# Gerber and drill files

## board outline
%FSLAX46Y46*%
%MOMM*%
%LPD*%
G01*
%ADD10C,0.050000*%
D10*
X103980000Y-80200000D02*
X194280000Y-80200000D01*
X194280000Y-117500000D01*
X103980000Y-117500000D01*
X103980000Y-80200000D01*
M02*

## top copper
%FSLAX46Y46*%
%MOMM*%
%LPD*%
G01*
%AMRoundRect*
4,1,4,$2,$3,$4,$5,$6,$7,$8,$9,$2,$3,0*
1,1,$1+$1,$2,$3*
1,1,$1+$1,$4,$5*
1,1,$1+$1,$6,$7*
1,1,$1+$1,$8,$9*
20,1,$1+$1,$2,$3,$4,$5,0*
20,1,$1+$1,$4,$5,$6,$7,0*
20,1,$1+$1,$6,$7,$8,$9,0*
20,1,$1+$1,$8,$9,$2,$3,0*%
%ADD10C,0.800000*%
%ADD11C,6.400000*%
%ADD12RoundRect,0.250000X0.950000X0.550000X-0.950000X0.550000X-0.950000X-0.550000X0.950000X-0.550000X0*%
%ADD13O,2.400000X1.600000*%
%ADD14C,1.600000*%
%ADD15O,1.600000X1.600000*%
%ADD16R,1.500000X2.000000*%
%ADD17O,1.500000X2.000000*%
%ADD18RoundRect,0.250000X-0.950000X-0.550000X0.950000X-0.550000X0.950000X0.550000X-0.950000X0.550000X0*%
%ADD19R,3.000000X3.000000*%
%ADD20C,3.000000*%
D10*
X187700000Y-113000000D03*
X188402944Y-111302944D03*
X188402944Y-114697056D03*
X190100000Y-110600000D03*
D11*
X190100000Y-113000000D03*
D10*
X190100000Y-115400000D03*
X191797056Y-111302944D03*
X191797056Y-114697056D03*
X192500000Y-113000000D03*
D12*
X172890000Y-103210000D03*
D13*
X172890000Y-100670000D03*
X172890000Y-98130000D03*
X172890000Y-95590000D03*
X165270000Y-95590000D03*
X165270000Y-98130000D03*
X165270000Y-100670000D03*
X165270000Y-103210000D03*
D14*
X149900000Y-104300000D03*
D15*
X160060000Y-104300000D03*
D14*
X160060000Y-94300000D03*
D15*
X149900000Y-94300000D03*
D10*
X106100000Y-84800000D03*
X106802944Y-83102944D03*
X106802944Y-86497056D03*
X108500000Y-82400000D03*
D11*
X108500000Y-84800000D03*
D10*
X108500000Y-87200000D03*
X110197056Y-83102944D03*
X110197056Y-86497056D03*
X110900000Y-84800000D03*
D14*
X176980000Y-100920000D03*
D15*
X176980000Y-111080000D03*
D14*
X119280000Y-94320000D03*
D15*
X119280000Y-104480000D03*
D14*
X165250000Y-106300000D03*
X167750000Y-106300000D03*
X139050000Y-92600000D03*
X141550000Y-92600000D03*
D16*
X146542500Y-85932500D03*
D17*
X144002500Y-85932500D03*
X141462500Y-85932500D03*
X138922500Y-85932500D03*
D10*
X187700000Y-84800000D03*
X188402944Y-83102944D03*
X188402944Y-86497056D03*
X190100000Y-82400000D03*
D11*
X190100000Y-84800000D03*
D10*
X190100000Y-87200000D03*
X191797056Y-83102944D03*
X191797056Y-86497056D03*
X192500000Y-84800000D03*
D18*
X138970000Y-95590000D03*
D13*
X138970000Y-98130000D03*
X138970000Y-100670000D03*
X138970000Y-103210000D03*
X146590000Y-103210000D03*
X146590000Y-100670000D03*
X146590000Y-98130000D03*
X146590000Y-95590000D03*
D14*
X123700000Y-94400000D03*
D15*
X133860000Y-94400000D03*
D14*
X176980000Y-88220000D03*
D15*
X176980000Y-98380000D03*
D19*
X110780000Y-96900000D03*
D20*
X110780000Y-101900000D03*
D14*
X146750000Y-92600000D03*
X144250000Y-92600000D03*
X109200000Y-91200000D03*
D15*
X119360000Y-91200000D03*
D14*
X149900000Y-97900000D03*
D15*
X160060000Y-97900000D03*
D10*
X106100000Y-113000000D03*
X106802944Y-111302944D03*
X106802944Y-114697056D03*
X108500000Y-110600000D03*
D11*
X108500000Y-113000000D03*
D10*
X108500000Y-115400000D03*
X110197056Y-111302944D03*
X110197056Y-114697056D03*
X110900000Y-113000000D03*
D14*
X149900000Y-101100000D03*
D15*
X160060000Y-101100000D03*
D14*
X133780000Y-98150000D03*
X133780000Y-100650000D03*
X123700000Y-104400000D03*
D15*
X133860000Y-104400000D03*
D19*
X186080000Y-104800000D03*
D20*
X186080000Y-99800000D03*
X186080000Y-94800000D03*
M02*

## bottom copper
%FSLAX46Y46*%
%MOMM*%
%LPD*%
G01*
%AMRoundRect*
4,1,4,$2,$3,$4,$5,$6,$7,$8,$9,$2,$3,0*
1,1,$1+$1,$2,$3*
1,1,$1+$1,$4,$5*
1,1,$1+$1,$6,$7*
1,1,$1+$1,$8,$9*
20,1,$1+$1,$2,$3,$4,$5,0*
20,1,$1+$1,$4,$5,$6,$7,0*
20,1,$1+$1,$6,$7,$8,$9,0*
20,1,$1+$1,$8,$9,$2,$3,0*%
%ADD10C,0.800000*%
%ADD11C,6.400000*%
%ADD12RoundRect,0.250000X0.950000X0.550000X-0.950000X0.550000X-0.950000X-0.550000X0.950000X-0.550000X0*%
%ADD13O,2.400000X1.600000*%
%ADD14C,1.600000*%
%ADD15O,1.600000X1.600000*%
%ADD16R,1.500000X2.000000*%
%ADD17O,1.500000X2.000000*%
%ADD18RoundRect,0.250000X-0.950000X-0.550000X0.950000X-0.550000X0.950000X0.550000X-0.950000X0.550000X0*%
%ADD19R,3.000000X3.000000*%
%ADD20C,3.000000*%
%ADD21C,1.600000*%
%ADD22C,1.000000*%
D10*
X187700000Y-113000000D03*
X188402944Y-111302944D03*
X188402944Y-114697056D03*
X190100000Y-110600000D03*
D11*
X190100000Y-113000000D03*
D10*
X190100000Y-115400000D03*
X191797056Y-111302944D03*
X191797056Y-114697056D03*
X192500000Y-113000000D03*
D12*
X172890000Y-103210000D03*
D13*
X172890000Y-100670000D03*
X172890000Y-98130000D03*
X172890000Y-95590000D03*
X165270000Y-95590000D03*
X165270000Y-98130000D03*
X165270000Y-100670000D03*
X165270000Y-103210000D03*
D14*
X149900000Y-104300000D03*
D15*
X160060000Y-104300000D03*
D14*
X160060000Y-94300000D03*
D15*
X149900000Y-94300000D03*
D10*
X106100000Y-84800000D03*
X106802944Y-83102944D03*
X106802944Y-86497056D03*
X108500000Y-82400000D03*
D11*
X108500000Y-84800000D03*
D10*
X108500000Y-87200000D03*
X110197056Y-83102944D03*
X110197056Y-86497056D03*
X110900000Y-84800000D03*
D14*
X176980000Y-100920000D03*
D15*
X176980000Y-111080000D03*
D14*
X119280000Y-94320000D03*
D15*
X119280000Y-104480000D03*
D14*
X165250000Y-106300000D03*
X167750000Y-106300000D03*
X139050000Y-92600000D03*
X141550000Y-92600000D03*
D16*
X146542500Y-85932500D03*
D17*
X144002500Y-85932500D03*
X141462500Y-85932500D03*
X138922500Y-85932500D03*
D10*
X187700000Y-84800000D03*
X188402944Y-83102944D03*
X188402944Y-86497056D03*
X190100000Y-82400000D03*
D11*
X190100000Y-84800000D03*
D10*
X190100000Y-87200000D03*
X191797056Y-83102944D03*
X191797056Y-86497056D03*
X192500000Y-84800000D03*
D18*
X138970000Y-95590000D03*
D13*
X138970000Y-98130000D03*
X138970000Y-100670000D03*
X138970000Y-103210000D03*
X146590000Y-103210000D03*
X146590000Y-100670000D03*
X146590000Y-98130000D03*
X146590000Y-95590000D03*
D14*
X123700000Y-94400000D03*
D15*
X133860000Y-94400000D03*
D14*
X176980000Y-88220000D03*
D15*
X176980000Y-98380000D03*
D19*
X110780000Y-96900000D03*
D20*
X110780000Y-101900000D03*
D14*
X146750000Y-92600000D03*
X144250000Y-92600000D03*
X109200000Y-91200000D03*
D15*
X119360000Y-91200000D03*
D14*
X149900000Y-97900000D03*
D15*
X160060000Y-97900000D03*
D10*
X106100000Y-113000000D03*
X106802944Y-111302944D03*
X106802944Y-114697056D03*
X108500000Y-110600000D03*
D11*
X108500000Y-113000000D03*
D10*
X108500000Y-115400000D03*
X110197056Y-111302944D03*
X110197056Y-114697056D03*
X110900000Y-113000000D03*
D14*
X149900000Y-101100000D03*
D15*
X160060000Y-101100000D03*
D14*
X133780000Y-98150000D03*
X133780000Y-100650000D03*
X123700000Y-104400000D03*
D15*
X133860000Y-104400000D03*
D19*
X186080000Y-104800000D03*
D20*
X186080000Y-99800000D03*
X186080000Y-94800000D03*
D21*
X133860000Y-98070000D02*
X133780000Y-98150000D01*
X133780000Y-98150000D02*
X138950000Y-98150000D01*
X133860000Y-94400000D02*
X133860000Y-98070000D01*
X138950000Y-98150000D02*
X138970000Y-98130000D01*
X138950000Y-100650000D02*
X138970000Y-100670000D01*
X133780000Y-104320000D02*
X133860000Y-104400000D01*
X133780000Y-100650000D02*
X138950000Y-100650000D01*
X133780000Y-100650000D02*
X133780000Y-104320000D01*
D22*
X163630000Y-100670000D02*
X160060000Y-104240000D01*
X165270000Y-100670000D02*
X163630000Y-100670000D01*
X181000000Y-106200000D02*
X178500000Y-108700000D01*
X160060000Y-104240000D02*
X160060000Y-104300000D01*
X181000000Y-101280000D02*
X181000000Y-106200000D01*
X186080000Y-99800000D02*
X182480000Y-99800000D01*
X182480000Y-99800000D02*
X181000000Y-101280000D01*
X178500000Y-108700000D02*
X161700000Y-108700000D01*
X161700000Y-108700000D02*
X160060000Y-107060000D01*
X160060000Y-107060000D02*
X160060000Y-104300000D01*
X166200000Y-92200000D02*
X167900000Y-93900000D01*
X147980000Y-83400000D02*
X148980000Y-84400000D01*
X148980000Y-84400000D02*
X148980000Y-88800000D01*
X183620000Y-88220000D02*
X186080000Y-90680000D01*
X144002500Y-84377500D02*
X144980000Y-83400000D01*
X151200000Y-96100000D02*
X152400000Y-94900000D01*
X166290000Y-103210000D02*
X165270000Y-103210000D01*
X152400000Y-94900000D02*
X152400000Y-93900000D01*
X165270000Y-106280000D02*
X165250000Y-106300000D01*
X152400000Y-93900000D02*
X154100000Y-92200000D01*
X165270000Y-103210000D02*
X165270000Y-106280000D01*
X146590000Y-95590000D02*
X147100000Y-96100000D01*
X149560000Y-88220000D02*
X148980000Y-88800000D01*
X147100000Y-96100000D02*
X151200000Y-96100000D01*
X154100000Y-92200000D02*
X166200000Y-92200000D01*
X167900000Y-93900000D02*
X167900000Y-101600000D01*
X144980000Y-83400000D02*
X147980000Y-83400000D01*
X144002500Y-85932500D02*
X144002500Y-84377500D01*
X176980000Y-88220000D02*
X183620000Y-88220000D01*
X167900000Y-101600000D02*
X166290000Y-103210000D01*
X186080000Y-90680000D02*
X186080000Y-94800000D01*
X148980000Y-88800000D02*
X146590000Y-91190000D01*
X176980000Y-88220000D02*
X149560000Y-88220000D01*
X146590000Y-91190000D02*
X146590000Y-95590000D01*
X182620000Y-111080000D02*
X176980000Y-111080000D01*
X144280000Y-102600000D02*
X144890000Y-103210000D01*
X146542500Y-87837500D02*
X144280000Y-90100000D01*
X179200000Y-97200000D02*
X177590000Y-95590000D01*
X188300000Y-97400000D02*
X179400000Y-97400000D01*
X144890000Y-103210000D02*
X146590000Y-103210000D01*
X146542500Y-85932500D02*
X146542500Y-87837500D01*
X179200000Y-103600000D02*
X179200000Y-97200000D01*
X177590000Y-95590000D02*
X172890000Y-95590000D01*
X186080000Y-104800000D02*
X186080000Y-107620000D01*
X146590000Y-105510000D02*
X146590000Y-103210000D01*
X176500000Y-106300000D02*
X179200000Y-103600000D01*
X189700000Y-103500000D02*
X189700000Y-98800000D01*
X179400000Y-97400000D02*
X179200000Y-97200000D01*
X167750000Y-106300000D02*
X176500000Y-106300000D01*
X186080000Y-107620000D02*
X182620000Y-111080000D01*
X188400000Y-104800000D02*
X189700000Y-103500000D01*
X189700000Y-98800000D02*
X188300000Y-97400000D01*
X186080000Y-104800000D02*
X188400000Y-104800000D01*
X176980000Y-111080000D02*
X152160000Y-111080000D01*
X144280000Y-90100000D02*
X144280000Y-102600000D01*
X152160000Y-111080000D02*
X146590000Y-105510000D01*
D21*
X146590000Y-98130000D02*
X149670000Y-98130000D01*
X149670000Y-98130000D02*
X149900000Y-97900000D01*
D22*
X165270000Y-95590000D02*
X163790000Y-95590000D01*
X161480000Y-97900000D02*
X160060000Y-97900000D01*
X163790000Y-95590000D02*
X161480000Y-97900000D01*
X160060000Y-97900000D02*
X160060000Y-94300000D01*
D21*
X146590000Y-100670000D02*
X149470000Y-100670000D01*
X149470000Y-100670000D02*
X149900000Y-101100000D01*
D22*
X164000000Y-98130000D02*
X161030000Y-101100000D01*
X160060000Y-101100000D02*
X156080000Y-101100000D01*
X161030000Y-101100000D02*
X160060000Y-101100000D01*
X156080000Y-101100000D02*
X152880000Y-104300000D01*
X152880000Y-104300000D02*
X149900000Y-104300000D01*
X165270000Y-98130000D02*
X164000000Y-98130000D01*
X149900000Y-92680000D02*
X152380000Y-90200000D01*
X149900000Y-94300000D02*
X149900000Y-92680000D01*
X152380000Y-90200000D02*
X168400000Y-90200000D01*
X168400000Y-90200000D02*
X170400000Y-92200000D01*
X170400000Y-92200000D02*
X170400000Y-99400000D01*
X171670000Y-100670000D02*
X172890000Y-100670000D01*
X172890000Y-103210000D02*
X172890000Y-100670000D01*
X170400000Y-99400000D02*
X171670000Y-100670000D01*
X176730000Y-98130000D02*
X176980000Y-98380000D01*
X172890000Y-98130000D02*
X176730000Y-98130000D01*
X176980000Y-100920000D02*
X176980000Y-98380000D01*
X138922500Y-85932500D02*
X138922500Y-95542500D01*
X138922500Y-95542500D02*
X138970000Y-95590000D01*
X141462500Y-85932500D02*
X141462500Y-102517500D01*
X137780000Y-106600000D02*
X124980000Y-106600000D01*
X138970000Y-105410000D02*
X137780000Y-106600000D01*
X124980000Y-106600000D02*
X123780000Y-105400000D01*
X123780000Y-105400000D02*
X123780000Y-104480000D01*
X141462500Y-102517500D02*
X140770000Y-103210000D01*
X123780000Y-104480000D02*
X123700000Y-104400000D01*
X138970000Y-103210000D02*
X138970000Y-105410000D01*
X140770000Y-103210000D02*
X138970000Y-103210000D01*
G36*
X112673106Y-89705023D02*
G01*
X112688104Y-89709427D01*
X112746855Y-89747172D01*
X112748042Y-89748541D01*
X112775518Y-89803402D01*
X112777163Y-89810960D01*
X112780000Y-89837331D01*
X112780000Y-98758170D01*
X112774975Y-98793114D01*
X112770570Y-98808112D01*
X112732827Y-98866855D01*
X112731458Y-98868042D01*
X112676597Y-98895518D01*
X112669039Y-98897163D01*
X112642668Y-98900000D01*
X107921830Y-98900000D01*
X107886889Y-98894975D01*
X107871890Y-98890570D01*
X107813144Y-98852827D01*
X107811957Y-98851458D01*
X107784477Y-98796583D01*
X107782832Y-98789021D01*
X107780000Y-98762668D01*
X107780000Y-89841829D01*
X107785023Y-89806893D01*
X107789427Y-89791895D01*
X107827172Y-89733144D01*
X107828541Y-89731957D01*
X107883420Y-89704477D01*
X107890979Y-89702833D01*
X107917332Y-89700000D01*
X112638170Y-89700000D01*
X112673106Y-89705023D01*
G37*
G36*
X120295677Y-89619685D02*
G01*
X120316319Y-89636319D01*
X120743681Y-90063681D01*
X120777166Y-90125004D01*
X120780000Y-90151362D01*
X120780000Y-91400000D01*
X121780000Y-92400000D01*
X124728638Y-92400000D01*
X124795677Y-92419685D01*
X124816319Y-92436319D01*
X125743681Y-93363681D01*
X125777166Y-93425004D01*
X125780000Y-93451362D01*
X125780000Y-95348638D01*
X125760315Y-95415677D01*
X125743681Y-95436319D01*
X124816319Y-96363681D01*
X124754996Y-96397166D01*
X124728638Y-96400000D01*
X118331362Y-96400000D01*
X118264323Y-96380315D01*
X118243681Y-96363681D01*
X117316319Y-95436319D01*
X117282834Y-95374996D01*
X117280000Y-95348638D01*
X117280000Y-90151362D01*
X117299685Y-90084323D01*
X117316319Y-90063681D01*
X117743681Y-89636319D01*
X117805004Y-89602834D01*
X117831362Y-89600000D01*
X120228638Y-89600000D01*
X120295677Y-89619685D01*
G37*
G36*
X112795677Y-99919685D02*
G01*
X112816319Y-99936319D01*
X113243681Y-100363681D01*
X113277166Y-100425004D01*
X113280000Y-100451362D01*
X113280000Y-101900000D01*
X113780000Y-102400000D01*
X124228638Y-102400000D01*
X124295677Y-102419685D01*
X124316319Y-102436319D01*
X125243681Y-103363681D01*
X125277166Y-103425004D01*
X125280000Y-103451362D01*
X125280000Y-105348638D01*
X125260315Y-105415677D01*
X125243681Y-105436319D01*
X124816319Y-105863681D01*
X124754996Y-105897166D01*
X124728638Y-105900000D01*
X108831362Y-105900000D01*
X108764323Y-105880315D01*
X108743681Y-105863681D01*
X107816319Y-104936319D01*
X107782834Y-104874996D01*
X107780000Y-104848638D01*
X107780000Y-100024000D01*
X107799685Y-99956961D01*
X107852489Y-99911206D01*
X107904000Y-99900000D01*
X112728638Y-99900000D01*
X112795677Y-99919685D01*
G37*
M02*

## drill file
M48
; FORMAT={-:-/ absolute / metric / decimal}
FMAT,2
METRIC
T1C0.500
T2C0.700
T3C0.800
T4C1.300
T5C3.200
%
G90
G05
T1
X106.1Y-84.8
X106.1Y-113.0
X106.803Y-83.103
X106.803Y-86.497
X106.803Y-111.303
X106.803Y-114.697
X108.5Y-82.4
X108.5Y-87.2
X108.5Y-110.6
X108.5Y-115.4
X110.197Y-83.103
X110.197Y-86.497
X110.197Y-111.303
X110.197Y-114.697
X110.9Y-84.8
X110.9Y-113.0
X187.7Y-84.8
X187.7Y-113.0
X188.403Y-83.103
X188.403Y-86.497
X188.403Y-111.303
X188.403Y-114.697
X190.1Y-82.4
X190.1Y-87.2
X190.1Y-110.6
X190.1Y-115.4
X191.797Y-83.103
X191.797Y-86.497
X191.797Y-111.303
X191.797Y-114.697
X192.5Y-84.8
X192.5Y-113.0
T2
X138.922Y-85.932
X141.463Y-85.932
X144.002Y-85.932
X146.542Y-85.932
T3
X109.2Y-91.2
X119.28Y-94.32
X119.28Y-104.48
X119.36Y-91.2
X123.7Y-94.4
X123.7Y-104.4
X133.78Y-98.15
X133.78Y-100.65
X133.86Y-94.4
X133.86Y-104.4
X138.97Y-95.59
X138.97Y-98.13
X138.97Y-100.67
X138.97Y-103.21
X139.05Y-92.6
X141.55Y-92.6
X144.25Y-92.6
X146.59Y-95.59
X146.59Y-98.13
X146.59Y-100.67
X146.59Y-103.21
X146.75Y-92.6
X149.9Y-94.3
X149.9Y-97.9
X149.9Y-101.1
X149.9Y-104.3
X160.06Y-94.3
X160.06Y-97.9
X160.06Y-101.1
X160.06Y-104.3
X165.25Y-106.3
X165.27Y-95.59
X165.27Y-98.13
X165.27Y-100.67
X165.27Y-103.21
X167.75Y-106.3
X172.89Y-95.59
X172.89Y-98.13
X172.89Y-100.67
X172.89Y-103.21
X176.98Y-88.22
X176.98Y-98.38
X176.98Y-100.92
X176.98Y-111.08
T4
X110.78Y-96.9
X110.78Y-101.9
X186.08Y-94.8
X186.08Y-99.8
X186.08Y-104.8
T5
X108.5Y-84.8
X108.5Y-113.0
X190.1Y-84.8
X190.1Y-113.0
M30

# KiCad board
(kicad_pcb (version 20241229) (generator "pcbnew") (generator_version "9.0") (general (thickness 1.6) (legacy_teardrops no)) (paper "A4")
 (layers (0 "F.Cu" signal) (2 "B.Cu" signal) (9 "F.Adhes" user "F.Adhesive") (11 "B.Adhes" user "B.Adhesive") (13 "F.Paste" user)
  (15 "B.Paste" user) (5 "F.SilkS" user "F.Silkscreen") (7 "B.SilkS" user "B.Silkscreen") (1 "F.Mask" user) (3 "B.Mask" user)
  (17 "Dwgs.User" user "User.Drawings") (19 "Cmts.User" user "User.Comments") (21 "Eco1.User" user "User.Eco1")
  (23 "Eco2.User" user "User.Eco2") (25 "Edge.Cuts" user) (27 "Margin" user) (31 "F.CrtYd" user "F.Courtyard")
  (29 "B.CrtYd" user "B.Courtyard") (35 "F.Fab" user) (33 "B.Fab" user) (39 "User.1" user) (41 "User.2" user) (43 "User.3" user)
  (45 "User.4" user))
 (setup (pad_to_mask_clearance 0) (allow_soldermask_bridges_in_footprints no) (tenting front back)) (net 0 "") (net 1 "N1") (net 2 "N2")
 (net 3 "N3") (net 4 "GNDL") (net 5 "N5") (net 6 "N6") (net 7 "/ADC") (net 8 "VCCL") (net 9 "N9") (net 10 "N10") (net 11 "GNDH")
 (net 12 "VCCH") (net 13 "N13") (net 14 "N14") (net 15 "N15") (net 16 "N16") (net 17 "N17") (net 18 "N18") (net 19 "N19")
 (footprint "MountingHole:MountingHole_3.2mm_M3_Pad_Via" (layer "F.Cu") (at 190.1 113)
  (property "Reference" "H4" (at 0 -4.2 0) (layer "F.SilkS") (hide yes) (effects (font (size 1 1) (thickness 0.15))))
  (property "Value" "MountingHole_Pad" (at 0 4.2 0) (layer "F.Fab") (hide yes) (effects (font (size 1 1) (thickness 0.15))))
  (pad "1" thru_hole circle (at -2.4 0) (size 0.8 0.8) (drill 0.5) (layers "*.Cu" "*.Mask") (remove_unused_layers no) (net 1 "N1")
   (zone_connect 2))
  (pad "1" thru_hole circle (at -1.697056 -1.697056) (size 0.8 0.8) (drill 0.5) (layers "*.Cu" "*.Mask") (remove_unused_layers no)
   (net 1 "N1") (zone_connect 2))
  (pad "1" thru_hole circle (at -1.697056 1.697056) (size 0.8 0.8) (drill 0.5) (layers "*.Cu" "*.Mask") (remove_unused_layers no)
   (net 1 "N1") (zone_connect 2))
  (pad "1" thru_hole circle (at 0 -2.4) (size 0.8 0.8) (drill 0.5) (layers "*.Cu" "*.Mask") (remove_unused_layers no) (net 1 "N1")
   (zone_connect 2))
  (pad "1" thru_hole circle (at 0 0) (size 6.4 6.4) (drill 3.2) (layers "*.Cu" "*.Mask") (remove_unused_layers no) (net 1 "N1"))
  (pad "1" thru_hole circle (at 0 2.4) (size 0.8 0.8) (drill 0.5) (layers "*.Cu" "*.Mask") (remove_unused_layers no) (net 1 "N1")
   (zone_connect 2))
  (pad "1" thru_hole circle (at 1.697056 -1.697056) (size 0.8 0.8) (drill 0.5) (layers "*.Cu" "*.Mask") (remove_unused_layers no)
   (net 1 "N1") (zone_connect 2))
  (pad "1" thru_hole circle (at 1.697056 1.697056) (size 0.8 0.8) (drill 0.5) (layers "*.Cu" "*.Mask") (remove_unused_layers no)
   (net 1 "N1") (zone_connect 2))
  (pad "1" thru_hole circle (at 2.4 0) (size 0.8 0.8) (drill 0.5) (layers "*.Cu" "*.Mask") (remove_unused_layers no) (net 1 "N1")
   (zone_connect 2)))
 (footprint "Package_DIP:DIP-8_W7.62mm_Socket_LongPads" (layer "F.Cu") (at 172.89 103.21 180)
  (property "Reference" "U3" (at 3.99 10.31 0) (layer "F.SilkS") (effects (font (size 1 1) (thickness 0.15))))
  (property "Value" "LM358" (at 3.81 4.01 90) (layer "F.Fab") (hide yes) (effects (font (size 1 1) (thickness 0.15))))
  (pad "1" thru_hole roundrect (at 0 0 180) (size 2.4 1.6) (drill 0.8) (layers "*.Cu" "*.Mask") (remove_unused_layers no)
   (roundrect_rratio 0.15625) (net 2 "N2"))
  (pad "2" thru_hole oval (at 0 2.54 180) (size 2.4 1.6) (drill 0.8) (layers "*.Cu" "*.Mask") (remove_unused_layers no) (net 2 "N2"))
  (pad "3" thru_hole oval (at 0 5.08 180) (size 2.4 1.6) (drill 0.8) (layers "*.Cu" "*.Mask") (remove_unused_layers no) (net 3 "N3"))
  (pad "4" thru_hole oval (at 0 7.62 180) (size 2.4 1.6) (drill 0.8) (layers "*.Cu" "*.Mask") (remove_unused_layers no) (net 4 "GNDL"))
  (pad "5" thru_hole oval (at 7.62 7.62 180) (size 2.4 1.6) (drill 0.8) (layers "*.Cu" "*.Mask") (remove_unused_layers no) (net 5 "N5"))
  (pad "6" thru_hole oval (at 7.62 5.08 180) (size 2.4 1.6) (drill 0.8) (layers "*.Cu" "*.Mask") (remove_unused_layers no) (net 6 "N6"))
  (pad "7" thru_hole oval (at 7.62 2.54 180) (size 2.4 1.6) (drill 0.8) (layers "*.Cu" "*.Mask") (remove_unused_layers no) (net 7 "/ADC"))
  (pad "8" thru_hole oval (at 7.62 0 180) (size 2.4 1.6) (drill 0.8) (layers "*.Cu" "*.Mask") (remove_unused_layers no) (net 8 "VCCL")))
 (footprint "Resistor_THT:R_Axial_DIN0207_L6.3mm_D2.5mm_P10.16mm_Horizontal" (layer "F.Cu") (at 149.9 104.3)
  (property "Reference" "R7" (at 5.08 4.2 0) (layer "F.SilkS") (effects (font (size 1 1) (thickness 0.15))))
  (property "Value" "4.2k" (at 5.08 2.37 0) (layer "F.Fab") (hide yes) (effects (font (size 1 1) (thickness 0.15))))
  (pad "1" thru_hole circle (at 0 0) (size 1.6 1.6) (drill 0.8) (layers "*.Cu" "*.Mask") (remove_unused_layers no) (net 6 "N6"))
  (pad "2" thru_hole oval (at 10.16 0) (size 1.6 1.6) (drill 0.8) (layers "*.Cu" "*.Mask") (remove_unused_layers no) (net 7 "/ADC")))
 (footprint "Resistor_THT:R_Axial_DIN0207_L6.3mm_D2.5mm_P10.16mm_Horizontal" (layer "F.Cu") (at 160.06 94.3 180)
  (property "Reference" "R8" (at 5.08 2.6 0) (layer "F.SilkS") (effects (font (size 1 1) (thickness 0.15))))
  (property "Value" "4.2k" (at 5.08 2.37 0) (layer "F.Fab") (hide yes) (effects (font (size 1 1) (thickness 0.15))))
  (pad "1" thru_hole circle (at 0 0 180) (size 1.6 1.6) (drill 0.8) (layers "*.Cu" "*.Mask") (remove_unused_layers no) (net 5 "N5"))
  (pad "2" thru_hole oval (at 10.16 0 180) (size 1.6 1.6) (drill 0.8) (layers "*.Cu" "*.Mask") (remove_unused_layers no) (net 2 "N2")))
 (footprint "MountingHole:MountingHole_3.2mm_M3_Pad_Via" (layer "F.Cu") (at 108.5 84.8)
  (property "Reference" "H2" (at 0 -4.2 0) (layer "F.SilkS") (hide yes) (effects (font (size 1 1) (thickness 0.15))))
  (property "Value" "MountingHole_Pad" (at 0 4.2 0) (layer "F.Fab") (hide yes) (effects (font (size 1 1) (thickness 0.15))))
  (pad "1" thru_hole circle (at -2.4 0) (size 0.8 0.8) (drill 0.5) (layers "*.Cu" "*.Mask") (remove_unused_layers no) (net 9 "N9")
   (zone_connect 2))
  (pad "1" thru_hole circle (at -1.697056 -1.697056) (size 0.8 0.8) (drill 0.5) (layers "*.Cu" "*.Mask") (remove_unused_layers no)
   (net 9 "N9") (zone_connect 2))
  (pad "1" thru_hole circle (at -1.697056 1.697056) (size 0.8 0.8) (drill 0.5) (layers "*.Cu" "*.Mask") (remove_unused_layers no)
   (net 9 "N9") (zone_connect 2))
  (pad "1" thru_hole circle (at 0 -2.4) (size 0.8 0.8) (drill 0.5) (layers "*.Cu" "*.Mask") (remove_unused_layers no) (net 9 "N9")
   (zone_connect 2))
  (pad "1" thru_hole circle (at 0 0) (size 6.4 6.4) (drill 3.2) (layers "*.Cu" "*.Mask") (remove_unused_layers no) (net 9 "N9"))
  (pad "1" thru_hole circle (at 0 2.4) (size 0.8 0.8) (drill 0.5) (layers "*.Cu" "*.Mask") (remove_unused_layers no) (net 9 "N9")
   (zone_connect 2))
  (pad "1" thru_hole circle (at 1.697056 -1.697056) (size 0.8 0.8) (drill 0.5) (layers "*.Cu" "*.Mask") (remove_unused_layers no)
   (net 9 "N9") (zone_connect 2))
  (pad "1" thru_hole circle (at 1.697056 1.697056) (size 0.8 0.8) (drill 0.5) (layers "*.Cu" "*.Mask") (remove_unused_layers no)
   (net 9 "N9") (zone_connect 2))
  (pad "1" thru_hole circle (at 2.4 0) (size 0.8 0.8) (drill 0.5) (layers "*.Cu" "*.Mask") (remove_unused_layers no) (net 9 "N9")
   (zone_connect 2)))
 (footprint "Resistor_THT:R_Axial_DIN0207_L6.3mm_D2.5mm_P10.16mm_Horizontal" (layer "F.Cu") (at 176.98 100.92 -90)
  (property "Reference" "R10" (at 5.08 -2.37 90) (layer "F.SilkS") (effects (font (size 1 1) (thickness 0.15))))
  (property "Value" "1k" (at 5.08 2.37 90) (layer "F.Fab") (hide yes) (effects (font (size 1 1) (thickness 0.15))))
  (pad "1" thru_hole circle (at 0 0 270) (size 1.6 1.6) (drill 0.8) (layers "*.Cu" "*.Mask") (remove_unused_layers no) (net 3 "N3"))
  (pad "2" thru_hole oval (at 10.16 0 270) (size 1.6 1.6) (drill 0.8) (layers "*.Cu" "*.Mask") (remove_unused_layers no) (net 4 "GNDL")))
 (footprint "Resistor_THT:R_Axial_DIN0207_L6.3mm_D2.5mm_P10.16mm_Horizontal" (layer "F.Cu") (at 119.28 94.32 -90)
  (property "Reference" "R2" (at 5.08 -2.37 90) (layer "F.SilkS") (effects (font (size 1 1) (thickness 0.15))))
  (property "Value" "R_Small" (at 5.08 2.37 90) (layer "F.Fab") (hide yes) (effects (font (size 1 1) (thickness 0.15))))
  (pad "1" thru_hole circle (at 0 0 270) (size 1.6 1.6) (drill 0.8) (layers "*.Cu" "*.Mask") (remove_unused_layers no) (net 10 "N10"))
  (pad "2" thru_hole oval (at 10.16 0 270) (size 1.6 1.6) (drill 0.8) (layers "*.Cu" "*.Mask") (remove_unused_layers no) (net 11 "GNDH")))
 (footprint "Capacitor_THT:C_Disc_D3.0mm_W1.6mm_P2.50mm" (layer "F.Cu") (at 165.25 106.3)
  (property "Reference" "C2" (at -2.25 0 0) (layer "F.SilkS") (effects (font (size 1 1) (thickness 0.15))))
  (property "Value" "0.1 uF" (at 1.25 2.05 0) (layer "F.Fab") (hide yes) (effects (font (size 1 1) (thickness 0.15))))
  (pad "1" thru_hole circle (at 0 0) (size 1.6 1.6) (drill 0.8) (layers "*.Cu" "*.Mask") (remove_unused_layers no) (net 8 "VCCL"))
  (pad "2" thru_hole circle (at 2.5 0) (size 1.6 1.6) (drill 0.8) (layers "*.Cu" "*.Mask") (remove_unused_layers no) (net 4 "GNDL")))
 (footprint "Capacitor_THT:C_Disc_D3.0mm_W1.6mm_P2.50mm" (layer "F.Cu") (at 139.05 92.6)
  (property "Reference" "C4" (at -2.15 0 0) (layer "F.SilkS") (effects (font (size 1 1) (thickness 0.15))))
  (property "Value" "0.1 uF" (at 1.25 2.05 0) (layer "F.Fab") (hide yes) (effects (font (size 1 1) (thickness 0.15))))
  (pad "1" thru_hole circle (at 0 0) (size 1.6 1.6) (drill 0.8) (layers "*.Cu" "*.Mask") (remove_unused_layers no) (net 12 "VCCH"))
  (pad "2" thru_hole circle (at 2.5 0) (size 1.6 1.6) (drill 0.8) (layers "*.Cu" "*.Mask") (remove_unused_layers no) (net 11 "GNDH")))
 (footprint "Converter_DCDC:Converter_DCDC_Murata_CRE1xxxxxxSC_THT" (layer "F.Cu") (at 146.5425 85.9325 -90)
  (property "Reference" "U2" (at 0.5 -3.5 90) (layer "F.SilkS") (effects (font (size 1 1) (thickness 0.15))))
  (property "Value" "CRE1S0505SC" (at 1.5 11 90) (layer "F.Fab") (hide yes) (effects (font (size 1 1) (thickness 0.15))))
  (pad "1" thru_hole rect (at 0 0 180) (size 1.5 2) (drill 0.7) (layers "*.Cu" "*.Mask") (remove_unused_layers no) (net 4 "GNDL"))
  (pad "2" thru_hole oval (at 0 2.54 180) (size 1.5 2) (drill 0.7) (layers "*.Cu" "*.Mask") (remove_unused_layers no) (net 8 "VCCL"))
  (pad "3" thru_hole oval (at 0 5.08 180) (size 1.5 2) (drill 0.7) (layers "*.Cu" "*.Mask") (remove_unused_layers no) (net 11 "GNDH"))
  (pad "4" thru_hole oval (at 0 7.62 180) (size 1.5 2) (drill 0.7) (layers "*.Cu" "*.Mask") (remove_unused_layers no) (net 12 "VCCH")))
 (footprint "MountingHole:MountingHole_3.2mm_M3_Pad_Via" (layer "F.Cu") (at 190.1 84.8)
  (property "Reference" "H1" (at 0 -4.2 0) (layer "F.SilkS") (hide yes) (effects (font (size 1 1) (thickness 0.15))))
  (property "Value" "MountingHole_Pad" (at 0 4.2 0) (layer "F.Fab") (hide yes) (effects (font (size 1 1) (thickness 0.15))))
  (pad "1" thru_hole circle (at -2.4 0) (size 0.8 0.8) (drill 0.5) (layers "*.Cu" "*.Mask") (remove_unused_layers no) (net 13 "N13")
   (zone_connect 2))
  (pad "1" thru_hole circle (at -1.697056 -1.697056) (size 0.8 0.8) (drill 0.5) (layers "*.Cu" "*.Mask") (remove_unused_layers no)
   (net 13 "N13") (zone_connect 2))
  (pad "1" thru_hole circle (at -1.697056 1.697056) (size 0.8 0.8) (drill 0.5) (layers "*.Cu" "*.Mask") (remove_unused_layers no)
   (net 13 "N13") (zone_connect 2))
  (pad "1" thru_hole circle (at 0 -2.4) (size 0.8 0.8) (drill 0.5) (layers "*.Cu" "*.Mask") (remove_unused_layers no) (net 13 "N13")
   (zone_connect 2))
  (pad "1" thru_hole circle (at 0 0) (size 6.4 6.4) (drill 3.2) (layers "*.Cu" "*.Mask") (remove_unused_layers no) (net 13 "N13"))
  (pad "1" thru_hole circle (at 0 2.4) (size 0.8 0.8) (drill 0.5) (layers "*.Cu" "*.Mask") (remove_unused_layers no) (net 13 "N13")
   (zone_connect 2))
  (pad "1" thru_hole circle (at 1.697056 -1.697056) (size 0.8 0.8) (drill 0.5) (layers "*.Cu" "*.Mask") (remove_unused_layers no)
   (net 13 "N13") (zone_connect 2))
  (pad "1" thru_hole circle (at 1.697056 1.697056) (size 0.8 0.8) (drill 0.5) (layers "*.Cu" "*.Mask") (remove_unused_layers no)
   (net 13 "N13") (zone_connect 2))
  (pad "1" thru_hole circle (at 2.4 0) (size 0.8 0.8) (drill 0.5) (layers "*.Cu" "*.Mask") (remove_unused_layers no) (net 13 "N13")
   (zone_connect 2)))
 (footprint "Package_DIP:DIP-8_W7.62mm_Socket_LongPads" (layer "F.Cu") (at 138.97 95.59)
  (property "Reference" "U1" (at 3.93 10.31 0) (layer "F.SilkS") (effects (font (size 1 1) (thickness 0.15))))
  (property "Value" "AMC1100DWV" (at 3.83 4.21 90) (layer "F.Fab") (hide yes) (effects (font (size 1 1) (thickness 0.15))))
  (pad "1" thru_hole roundrect (at 0 0) (size 2.4 1.6) (drill 0.8) (layers "*.Cu" "*.Mask") (remove_unused_layers no)
   (roundrect_rratio 0.15625) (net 12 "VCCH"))
  (pad "2" thru_hole oval (at 0 2.54) (size 2.4 1.6) (drill 0.8) (layers "*.Cu" "*.Mask") (remove_unused_layers no) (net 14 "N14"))
  (pad "3" thru_hole oval (at 0 5.08) (size 2.4 1.6) (drill 0.8) (layers "*.Cu" "*.Mask") (remove_unused_layers no) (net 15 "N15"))
  (pad "4" thru_hole oval (at 0 7.62) (size 2.4 1.6) (drill 0.8) (layers "*.Cu" "*.Mask") (remove_unused_layers no) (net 11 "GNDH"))
  (pad "5" thru_hole oval (at 7.62 7.62) (size 2.4 1.6) (drill 0.8) (layers "*.Cu" "*.Mask") (remove_unused_layers no) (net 4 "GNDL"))
  (pad "6" thru_hole oval (at 7.62 5.08) (size 2.4 1.6) (drill 0.8) (layers "*.Cu" "*.Mask") (remove_unused_layers no) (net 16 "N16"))
  (pad "7" thru_hole oval (at 7.62 2.54) (size 2.4 1.6) (drill 0.8) (layers "*.Cu" "*.Mask") (remove_unused_layers no) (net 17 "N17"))
  (pad "8" thru_hole oval (at 7.62 0) (size 2.4 1.6) (drill 0.8) (layers "*.Cu" "*.Mask") (remove_unused_layers no) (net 8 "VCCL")))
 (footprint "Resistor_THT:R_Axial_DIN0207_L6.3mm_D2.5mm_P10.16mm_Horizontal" (layer "F.Cu") (at 123.7 94.4)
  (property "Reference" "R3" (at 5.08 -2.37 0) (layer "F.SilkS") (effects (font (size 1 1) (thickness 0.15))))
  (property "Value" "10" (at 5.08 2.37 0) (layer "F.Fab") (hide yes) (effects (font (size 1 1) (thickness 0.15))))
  (pad "1" thru_hole circle (at 0 0) (size 1.6 1.6) (drill 0.8) (layers "*.Cu" "*.Mask") (remove_unused_layers no) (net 10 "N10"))
  (pad "2" thru_hole oval (at 10.16 0) (size 1.6 1.6) (drill 0.8) (layers "*.Cu" "*.Mask") (remove_unused_layers no) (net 14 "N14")))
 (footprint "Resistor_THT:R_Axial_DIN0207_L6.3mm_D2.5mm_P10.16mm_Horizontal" (layer "F.Cu") (at 176.98 88.22 -90)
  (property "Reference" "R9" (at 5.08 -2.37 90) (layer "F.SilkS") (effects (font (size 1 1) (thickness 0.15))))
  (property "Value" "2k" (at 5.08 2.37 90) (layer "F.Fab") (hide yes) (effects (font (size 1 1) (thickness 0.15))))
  (pad "1" thru_hole circle (at 0 0 270) (size 1.6 1.6) (drill 0.8) (layers "*.Cu" "*.Mask") (remove_unused_layers no) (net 8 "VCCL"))
  (pad "2" thru_hole oval (at 10.16 0 270) (size 1.6 1.6) (drill 0.8) (layers "*.Cu" "*.Mask") (remove_unused_layers no) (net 3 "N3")))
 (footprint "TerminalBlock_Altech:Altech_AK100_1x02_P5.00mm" (layer "F.Cu") (at 110.78 96.9 -90)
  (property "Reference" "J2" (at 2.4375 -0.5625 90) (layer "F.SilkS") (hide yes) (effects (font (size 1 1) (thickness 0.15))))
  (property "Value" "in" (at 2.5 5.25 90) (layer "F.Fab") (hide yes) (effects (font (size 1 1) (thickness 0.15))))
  (pad "1" thru_hole rect (at 0 0 270) (size 3 3) (drill 1.3) (layers "*.Cu" "*.Mask") (remove_unused_layers no) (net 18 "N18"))
  (pad "2" thru_hole circle (at 5 0 270) (size 3 3) (drill 1.3) (layers "*.Cu" "*.Mask") (remove_unused_layers no) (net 11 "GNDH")))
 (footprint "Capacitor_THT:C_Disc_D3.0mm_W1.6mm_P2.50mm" (layer "F.Cu") (at 146.75 92.6 180)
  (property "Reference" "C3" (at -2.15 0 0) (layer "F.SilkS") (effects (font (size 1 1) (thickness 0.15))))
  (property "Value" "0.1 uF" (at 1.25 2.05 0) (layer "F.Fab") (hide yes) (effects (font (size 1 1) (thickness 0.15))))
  (pad "1" thru_hole circle (at 0 0 180) (size 1.6 1.6) (drill 0.8) (layers "*.Cu" "*.Mask") (remove_unused_layers no) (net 8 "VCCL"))
  (pad "2" thru_hole circle (at 2.5 0 180) (size 1.6 1.6) (drill 0.8) (layers "*.Cu" "*.Mask") (remove_unused_layers no) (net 4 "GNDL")))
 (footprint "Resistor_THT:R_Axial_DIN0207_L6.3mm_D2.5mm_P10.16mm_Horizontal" (layer "F.Cu") (at 109.2 91.2)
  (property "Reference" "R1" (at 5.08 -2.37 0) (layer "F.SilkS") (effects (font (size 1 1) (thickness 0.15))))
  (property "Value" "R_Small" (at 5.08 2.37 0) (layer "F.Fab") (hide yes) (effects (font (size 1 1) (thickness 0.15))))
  (pad "1" thru_hole circle (at 0 0) (size 1.6 1.6) (drill 0.8) (layers "*.Cu" "*.Mask") (remove_unused_layers no) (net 18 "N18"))
  (pad "2" thru_hole oval (at 10.16 0) (size 1.6 1.6) (drill 0.8) (layers "*.Cu" "*.Mask") (remove_unused_layers no) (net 10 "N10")))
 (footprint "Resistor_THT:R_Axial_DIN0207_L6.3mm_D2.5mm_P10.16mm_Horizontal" (layer "F.Cu") (at 149.9 97.9)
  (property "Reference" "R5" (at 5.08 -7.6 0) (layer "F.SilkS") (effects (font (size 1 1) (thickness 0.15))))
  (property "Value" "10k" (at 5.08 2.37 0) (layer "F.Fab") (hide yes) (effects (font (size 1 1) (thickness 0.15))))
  (pad "1" thru_hole circle (at 0 0) (size 1.6 1.6) (drill 0.8) (layers "*.Cu" "*.Mask") (remove_unused_layers no) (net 17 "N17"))
  (pad "2" thru_hole oval (at 10.16 0) (size 1.6 1.6) (drill 0.8) (layers "*.Cu" "*.Mask") (remove_unused_layers no) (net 5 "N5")))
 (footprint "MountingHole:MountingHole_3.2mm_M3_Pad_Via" (layer "F.Cu") (at 108.5 113)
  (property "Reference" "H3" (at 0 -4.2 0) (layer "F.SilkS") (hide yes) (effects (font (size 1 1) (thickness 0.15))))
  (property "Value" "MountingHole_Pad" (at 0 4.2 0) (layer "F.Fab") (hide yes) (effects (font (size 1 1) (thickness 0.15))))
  (pad "1" thru_hole circle (at -2.4 0) (size 0.8 0.8) (drill 0.5) (layers "*.Cu" "*.Mask") (remove_unused_layers no) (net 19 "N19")
   (zone_connect 2))
  (pad "1" thru_hole circle (at -1.697056 -1.697056) (size 0.8 0.8) (drill 0.5) (layers "*.Cu" "*.Mask") (remove_unused_layers no)
   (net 19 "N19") (zone_connect 2))
  (pad "1" thru_hole circle (at -1.697056 1.697056) (size 0.8 0.8) (drill 0.5) (layers "*.Cu" "*.Mask") (remove_unused_layers no)
   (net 19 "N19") (zone_connect 2))
  (pad "1" thru_hole circle (at 0 -2.4) (size 0.8 0.8) (drill 0.5) (layers "*.Cu" "*.Mask") (remove_unused_layers no) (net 19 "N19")
   (zone_connect 2))
  (pad "1" thru_hole circle (at 0 0) (size 6.4 6.4) (drill 3.2) (layers "*.Cu" "*.Mask") (remove_unused_layers no) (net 19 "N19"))
  (pad "1" thru_hole circle (at 0 2.4) (size 0.8 0.8) (drill 0.5) (layers "*.Cu" "*.Mask") (remove_unused_layers no) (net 19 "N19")
   (zone_connect 2))
  (pad "1" thru_hole circle (at 1.697056 -1.697056) (size 0.8 0.8) (drill 0.5) (layers "*.Cu" "*.Mask") (remove_unused_layers no)
   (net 19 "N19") (zone_connect 2))
  (pad "1" thru_hole circle (at 1.697056 1.697056) (size 0.8 0.8) (drill 0.5) (layers "*.Cu" "*.Mask") (remove_unused_layers no)
   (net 19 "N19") (zone_connect 2))
  (pad "1" thru_hole circle (at 2.4 0) (size 0.8 0.8) (drill 0.5) (layers "*.Cu" "*.Mask") (remove_unused_layers no) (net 19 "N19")
   (zone_connect 2)))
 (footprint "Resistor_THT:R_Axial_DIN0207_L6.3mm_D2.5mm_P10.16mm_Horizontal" (layer "F.Cu") (at 149.9 101.1)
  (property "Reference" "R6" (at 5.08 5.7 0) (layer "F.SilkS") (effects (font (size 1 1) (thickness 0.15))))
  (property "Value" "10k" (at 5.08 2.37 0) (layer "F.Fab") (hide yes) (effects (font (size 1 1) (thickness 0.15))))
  (pad "1" thru_hole circle (at 0 0) (size 1.6 1.6) (drill 0.8) (layers "*.Cu" "*.Mask") (remove_unused_layers no) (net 16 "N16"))
  (pad "2" thru_hole oval (at 10.16 0) (size 1.6 1.6) (drill 0.8) (layers "*.Cu" "*.Mask") (remove_unused_layers no) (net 6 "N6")))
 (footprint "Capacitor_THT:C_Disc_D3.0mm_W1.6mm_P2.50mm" (layer "F.Cu") (at 133.78 98.15 -90)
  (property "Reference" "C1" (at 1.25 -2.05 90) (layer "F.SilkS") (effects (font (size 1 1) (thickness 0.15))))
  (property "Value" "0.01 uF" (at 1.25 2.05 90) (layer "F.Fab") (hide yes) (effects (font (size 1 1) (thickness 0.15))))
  (pad "1" thru_hole circle (at 0 0 270) (size 1.6 1.6) (drill 0.8) (layers "*.Cu" "*.Mask") (remove_unused_layers no) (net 14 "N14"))
  (pad "2" thru_hole circle (at 2.5 0 270) (size 1.6 1.6) (drill 0.8) (layers "*.Cu" "*.Mask") (remove_unused_layers no) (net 15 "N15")))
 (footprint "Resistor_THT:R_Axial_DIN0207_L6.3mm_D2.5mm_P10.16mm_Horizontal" (layer "F.Cu") (at 123.7 104.4)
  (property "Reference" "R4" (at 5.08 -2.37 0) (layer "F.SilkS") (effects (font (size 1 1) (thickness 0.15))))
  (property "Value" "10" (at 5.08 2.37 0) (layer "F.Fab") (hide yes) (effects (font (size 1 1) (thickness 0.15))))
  (pad "1" thru_hole circle (at 0 0) (size 1.6 1.6) (drill 0.8) (layers "*.Cu" "*.Mask") (remove_unused_layers no) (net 11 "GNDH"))
  (pad "2" thru_hole oval (at 10.16 0) (size 1.6 1.6) (drill 0.8) (layers "*.Cu" "*.Mask") (remove_unused_layers no) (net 15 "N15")))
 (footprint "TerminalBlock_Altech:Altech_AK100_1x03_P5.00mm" (layer "F.Cu") (at 186.08 104.8 90)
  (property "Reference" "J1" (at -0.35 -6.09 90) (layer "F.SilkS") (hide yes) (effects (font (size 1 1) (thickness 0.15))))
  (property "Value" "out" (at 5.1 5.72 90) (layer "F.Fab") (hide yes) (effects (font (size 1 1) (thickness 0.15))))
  (pad "1" thru_hole rect (at 0 0 90) (size 3 3) (drill 1.3) (layers "*.Cu" "*.Mask") (remove_unused_layers no) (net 4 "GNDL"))
  (pad "2" thru_hole circle (at 5 0 90) (size 3 3) (drill 1.3) (layers "*.Cu" "*.Mask") (remove_unused_layers no) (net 7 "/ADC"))
  (pad "3" thru_hole circle (at 10 0 90) (size 3 3) (drill 1.3) (layers "*.Cu" "*.Mask") (remove_unused_layers no) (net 8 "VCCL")))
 (gr_rect (start 103.98 80.2) (end 194.28 117.5) (stroke (width 0.05) (type default)) (fill no) (layer "Edge.Cuts"))
 (segment (start 133.86 98.07) (end 133.78 98.15) (width 1.6) (layer "B.Cu") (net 14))
 (segment (start 133.78 98.15) (end 138.95 98.15) (width 1.6) (layer "B.Cu") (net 14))
 (segment (start 133.86 94.4) (end 133.86 98.07) (width 1.6) (layer "B.Cu") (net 14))
 (segment (start 138.95 98.15) (end 138.97 98.13) (width 1.6) (layer "B.Cu") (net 14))
 (segment (start 138.95 100.65) (end 138.97 100.67) (width 1.6) (layer "B.Cu") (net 15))
 (segment (start 133.78 104.32) (end 133.86 104.4) (width 1.6) (layer "B.Cu") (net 15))
 (segment (start 133.78 100.65) (end 138.95 100.65) (width 1.6) (layer "B.Cu") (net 15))
 (segment (start 133.78 100.65) (end 133.78 104.32) (width 1.6) (layer "B.Cu") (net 15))
 (segment (start 163.63 100.67) (end 160.06 104.24) (width 1) (layer "B.Cu") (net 7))
 (segment (start 165.27 100.67) (end 163.63 100.67) (width 1) (layer "B.Cu") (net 7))
 (segment (start 181 106.2) (end 178.5 108.7) (width 1) (layer "B.Cu") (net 7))
 (segment (start 160.06 104.24) (end 160.06 104.3) (width 1) (layer "B.Cu") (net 7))
 (segment (start 181 101.28) (end 181 106.2) (width 1) (layer "B.Cu") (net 7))
 (segment (start 186.08 99.8) (end 182.48 99.8) (width 1) (layer "B.Cu") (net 7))
 (segment (start 182.48 99.8) (end 181 101.28) (width 1) (layer "B.Cu") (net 7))
 (segment (start 178.5 108.7) (end 161.7 108.7) (width 1) (layer "B.Cu") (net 7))
 (segment (start 161.7 108.7) (end 160.06 107.06) (width 1) (layer "B.Cu") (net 7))
 (segment (start 160.06 107.06) (end 160.06 104.3) (width 1) (layer "B.Cu") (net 7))
 (segment (start 166.2 92.2) (end 167.9 93.9) (width 1) (layer "B.Cu") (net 8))
 (segment (start 147.98 83.4) (end 148.98 84.4) (width 1) (layer "B.Cu") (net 8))
 (segment (start 148.98 84.4) (end 148.98 88.8) (width 1) (layer "B.Cu") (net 8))
 (segment (start 183.62 88.22) (end 186.08 90.68) (width 1) (layer "B.Cu") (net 8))
 (segment (start 144.0025 84.3775) (end 144.98 83.4) (width 1) (layer "B.Cu") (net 8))
 (segment (start 151.2 96.1) (end 152.4 94.9) (width 1) (layer "B.Cu") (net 8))
 (segment (start 166.29 103.21) (end 165.27 103.21) (width 1) (layer "B.Cu") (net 8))
 (segment (start 152.4 94.9) (end 152.4 93.9) (width 1) (layer "B.Cu") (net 8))
 (segment (start 165.27 106.28) (end 165.25 106.3) (width 1) (layer "B.Cu") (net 8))
 (segment (start 152.4 93.9) (end 154.1 92.2) (width 1) (layer "B.Cu") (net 8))
 (segment (start 165.27 103.21) (end 165.27 106.28) (width 1) (layer "B.Cu") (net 8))
 (segment (start 146.59 95.59) (end 147.1 96.1) (width 1) (layer "B.Cu") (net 8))
 (segment (start 149.56 88.22) (end 148.98 88.8) (width 1) (layer "B.Cu") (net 8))
 (segment (start 147.1 96.1) (end 151.2 96.1) (width 1) (layer "B.Cu") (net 8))
 (segment (start 154.1 92.2) (end 166.2 92.2) (width 1) (layer "B.Cu") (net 8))
 (segment (start 167.9 93.9) (end 167.9 101.6) (width 1) (layer "B.Cu") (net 8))
 (segment (start 144.98 83.4) (end 147.98 83.4) (width 1) (layer "B.Cu") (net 8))
 (segment (start 144.0025 85.9325) (end 144.0025 84.3775) (width 1) (layer "B.Cu") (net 8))
 (segment (start 176.98 88.22) (end 183.62 88.22) (width 1) (layer "B.Cu") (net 8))
 (segment (start 167.9 101.6) (end 166.29 103.21) (width 1) (layer "B.Cu") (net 8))
 (segment (start 186.08 90.68) (end 186.08 94.8) (width 1) (layer "B.Cu") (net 8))
 (segment (start 148.98 88.8) (end 146.59 91.19) (width 1) (layer "B.Cu") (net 8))
 (segment (start 176.98 88.22) (end 149.56 88.22) (width 1) (layer "B.Cu") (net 8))
 (segment (start 146.59 91.19) (end 146.59 95.59) (width 1) (layer "B.Cu") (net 8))
 (segment (start 182.62 111.08) (end 176.98 111.08) (width 1) (layer "B.Cu") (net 4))
 (segment (start 144.28 102.6) (end 144.89 103.21) (width 1) (layer "B.Cu") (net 4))
 (segment (start 146.5425 87.8375) (end 144.28 90.1) (width 1) (layer "B.Cu") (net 4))
 (segment (start 179.2 97.2) (end 177.59 95.59) (width 1) (layer "B.Cu") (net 4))
 (segment (start 188.3 97.4) (end 179.4 97.4) (width 1) (layer "B.Cu") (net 4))
 (segment (start 144.89 103.21) (end 146.59 103.21) (width 1) (layer "B.Cu") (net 4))
 (segment (start 146.5425 85.9325) (end 146.5425 87.8375) (width 1) (layer "B.Cu") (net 4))
 (segment (start 179.2 103.6) (end 179.2 97.2) (width 1) (layer "B.Cu") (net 4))
 (segment (start 177.59 95.59) (end 172.89 95.59) (width 1) (layer "B.Cu") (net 4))
 (segment (start 186.08 104.8) (end 186.08 107.62) (width 1) (layer "B.Cu") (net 4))
 (segment (start 146.59 105.51) (end 146.59 103.21) (width 1) (layer "B.Cu") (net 4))
 (segment (start 176.5 106.3) (end 179.2 103.6) (width 1) (layer "B.Cu") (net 4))
 (segment (start 189.7 103.5) (end 189.7 98.8) (width 1) (layer "B.Cu") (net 4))
 (segment (start 179.4 97.4) (end 179.2 97.2) (width 1) (layer "B.Cu") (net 4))
 (segment (start 167.75 106.3) (end 176.5 106.3) (width 1) (layer "B.Cu") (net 4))
 (segment (start 186.08 107.62) (end 182.62 111.08) (width 1) (layer "B.Cu") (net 4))
 (segment (start 188.4 104.8) (end 189.7 103.5) (width 1) (layer "B.Cu") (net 4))
 (segment (start 189.7 98.8) (end 188.3 97.4) (width 1) (layer "B.Cu") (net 4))
 (segment (start 186.08 104.8) (end 188.4 104.8) (width 1) (layer "B.Cu") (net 4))
 (segment (start 176.98 111.08) (end 152.16 111.08) (width 1) (layer "B.Cu") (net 4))
 (segment (start 144.28 90.1) (end 144.28 102.6) (width 1) (layer "B.Cu") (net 4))
 (segment (start 152.16 111.08) (end 146.59 105.51) (width 1) (layer "B.Cu") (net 4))
 (segment (start 146.59 98.13) (end 149.67 98.13) (width 1.6) (layer "B.Cu") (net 17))
 (segment (start 149.67 98.13) (end 149.9 97.9) (width 1.6) (layer "B.Cu") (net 17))
 (segment (start 165.27 95.59) (end 163.79 95.59) (width 1) (layer "B.Cu") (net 5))
 (segment (start 161.48 97.9) (end 160.06 97.9) (width 1) (layer "B.Cu") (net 5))
 (segment (start 163.79 95.59) (end 161.48 97.9) (width 1) (layer "B.Cu") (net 5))
 (segment (start 160.06 97.9) (end 160.06 94.3) (width 1) (layer "B.Cu") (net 5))
 (segment (start 146.59 100.67) (end 149.47 100.67) (width 1.6) (layer "B.Cu") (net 16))
 (segment (start 149.47 100.67) (end 149.9 101.1) (width 1.6) (layer "B.Cu") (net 16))
 (segment (start 164 98.13) (end 161.03 101.1) (width 1) (layer "B.Cu") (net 6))
 (segment (start 160.06 101.1) (end 156.08 101.1) (width 1) (layer "B.Cu") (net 6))
 (segment (start 161.03 101.1) (end 160.06 101.1) (width 1) (layer "B.Cu") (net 6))
 (segment (start 156.08 101.1) (end 152.88 104.3) (width 1) (layer "B.Cu") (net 6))
 (segment (start 152.88 104.3) (end 149.9 104.3) (width 1) (layer "B.Cu") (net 6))
 (segment (start 165.27 98.13) (end 164 98.13) (width 1) (layer "B.Cu") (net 6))
 (segment (start 149.9 92.68) (end 152.38 90.2) (width 1) (layer "B.Cu") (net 2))
 (segment (start 149.9 94.3) (end 149.9 92.68) (width 1) (layer "B.Cu") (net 2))
 (segment (start 152.38 90.2) (end 168.4 90.2) (width 1) (layer "B.Cu") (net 2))
 (segment (start 168.4 90.2) (end 170.4 92.2) (width 1) (layer "B.Cu") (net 2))
 (segment (start 170.4 92.2) (end 170.4 99.4) (width 1) (layer "B.Cu") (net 2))
 (segment (start 171.67 100.67) (end 172.89 100.67) (width 1) (layer "B.Cu") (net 2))
 (segment (start 172.89 103.21) (end 172.89 100.67) (width 1) (layer "B.Cu") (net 2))
 (segment (start 170.4 99.4) (end 171.67 100.67) (width 1) (layer "B.Cu") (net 2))
 (segment (start 176.73 98.13) (end 176.98 98.38) (width 1) (layer "B.Cu") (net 3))
 (segment (start 172.89 98.13) (end 176.73 98.13) (width 1) (layer "B.Cu") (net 3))
 (segment (start 176.98 100.92) (end 176.98 98.38) (width 1) (layer "B.Cu") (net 3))
 (segment (start 138.9225 85.9325) (end 138.9225 95.5425) (width 1) (layer "B.Cu") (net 12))
 (segment (start 138.9225 95.5425) (end 138.97 95.59) (width 1) (layer "B.Cu") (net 12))
 (segment (start 141.4625 85.9325) (end 141.4625 102.5175) (width 1) (layer "B.Cu") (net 11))
 (segment (start 137.78 106.6) (end 124.98 106.6) (width 1) (layer "B.Cu") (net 11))
 (segment (start 138.97 105.41) (end 137.78 106.6) (width 1) (layer "B.Cu") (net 11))
 (segment (start 124.98 106.6) (end 123.78 105.4) (width 1) (layer "B.Cu") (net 11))
 (segment (start 123.78 105.4) (end 123.78 104.48) (width 1) (layer "B.Cu") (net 11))
 (segment (start 141.4625 102.5175) (end 140.77 103.21) (width 1) (layer "B.Cu") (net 11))
 (segment (start 123.78 104.48) (end 123.7 104.4) (width 1) (layer "B.Cu") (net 11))
 (segment (start 138.97 103.21) (end 138.97 105.41) (width 1) (layer "B.Cu") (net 11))
 (segment (start 140.77 103.21) (end 138.97 103.21) (width 1) (layer "B.Cu") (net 11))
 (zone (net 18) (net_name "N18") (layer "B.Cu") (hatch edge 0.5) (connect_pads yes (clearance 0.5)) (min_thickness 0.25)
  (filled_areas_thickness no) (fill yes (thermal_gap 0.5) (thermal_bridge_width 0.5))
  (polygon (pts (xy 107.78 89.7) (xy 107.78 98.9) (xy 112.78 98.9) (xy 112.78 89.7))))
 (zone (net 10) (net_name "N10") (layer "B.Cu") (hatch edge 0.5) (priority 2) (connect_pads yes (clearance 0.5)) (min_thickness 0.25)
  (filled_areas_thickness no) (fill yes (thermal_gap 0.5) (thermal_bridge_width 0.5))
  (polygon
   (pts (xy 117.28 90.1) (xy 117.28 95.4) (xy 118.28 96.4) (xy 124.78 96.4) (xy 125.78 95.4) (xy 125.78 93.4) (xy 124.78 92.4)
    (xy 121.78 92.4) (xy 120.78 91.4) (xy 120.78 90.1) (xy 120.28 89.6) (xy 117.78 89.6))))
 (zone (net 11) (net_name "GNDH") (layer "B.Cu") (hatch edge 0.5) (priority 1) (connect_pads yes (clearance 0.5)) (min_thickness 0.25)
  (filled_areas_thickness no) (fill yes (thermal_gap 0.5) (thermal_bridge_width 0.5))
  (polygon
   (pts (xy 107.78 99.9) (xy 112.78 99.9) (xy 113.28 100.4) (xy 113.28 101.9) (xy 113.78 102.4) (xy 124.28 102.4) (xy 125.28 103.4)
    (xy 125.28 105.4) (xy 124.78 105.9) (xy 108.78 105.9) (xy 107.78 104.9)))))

